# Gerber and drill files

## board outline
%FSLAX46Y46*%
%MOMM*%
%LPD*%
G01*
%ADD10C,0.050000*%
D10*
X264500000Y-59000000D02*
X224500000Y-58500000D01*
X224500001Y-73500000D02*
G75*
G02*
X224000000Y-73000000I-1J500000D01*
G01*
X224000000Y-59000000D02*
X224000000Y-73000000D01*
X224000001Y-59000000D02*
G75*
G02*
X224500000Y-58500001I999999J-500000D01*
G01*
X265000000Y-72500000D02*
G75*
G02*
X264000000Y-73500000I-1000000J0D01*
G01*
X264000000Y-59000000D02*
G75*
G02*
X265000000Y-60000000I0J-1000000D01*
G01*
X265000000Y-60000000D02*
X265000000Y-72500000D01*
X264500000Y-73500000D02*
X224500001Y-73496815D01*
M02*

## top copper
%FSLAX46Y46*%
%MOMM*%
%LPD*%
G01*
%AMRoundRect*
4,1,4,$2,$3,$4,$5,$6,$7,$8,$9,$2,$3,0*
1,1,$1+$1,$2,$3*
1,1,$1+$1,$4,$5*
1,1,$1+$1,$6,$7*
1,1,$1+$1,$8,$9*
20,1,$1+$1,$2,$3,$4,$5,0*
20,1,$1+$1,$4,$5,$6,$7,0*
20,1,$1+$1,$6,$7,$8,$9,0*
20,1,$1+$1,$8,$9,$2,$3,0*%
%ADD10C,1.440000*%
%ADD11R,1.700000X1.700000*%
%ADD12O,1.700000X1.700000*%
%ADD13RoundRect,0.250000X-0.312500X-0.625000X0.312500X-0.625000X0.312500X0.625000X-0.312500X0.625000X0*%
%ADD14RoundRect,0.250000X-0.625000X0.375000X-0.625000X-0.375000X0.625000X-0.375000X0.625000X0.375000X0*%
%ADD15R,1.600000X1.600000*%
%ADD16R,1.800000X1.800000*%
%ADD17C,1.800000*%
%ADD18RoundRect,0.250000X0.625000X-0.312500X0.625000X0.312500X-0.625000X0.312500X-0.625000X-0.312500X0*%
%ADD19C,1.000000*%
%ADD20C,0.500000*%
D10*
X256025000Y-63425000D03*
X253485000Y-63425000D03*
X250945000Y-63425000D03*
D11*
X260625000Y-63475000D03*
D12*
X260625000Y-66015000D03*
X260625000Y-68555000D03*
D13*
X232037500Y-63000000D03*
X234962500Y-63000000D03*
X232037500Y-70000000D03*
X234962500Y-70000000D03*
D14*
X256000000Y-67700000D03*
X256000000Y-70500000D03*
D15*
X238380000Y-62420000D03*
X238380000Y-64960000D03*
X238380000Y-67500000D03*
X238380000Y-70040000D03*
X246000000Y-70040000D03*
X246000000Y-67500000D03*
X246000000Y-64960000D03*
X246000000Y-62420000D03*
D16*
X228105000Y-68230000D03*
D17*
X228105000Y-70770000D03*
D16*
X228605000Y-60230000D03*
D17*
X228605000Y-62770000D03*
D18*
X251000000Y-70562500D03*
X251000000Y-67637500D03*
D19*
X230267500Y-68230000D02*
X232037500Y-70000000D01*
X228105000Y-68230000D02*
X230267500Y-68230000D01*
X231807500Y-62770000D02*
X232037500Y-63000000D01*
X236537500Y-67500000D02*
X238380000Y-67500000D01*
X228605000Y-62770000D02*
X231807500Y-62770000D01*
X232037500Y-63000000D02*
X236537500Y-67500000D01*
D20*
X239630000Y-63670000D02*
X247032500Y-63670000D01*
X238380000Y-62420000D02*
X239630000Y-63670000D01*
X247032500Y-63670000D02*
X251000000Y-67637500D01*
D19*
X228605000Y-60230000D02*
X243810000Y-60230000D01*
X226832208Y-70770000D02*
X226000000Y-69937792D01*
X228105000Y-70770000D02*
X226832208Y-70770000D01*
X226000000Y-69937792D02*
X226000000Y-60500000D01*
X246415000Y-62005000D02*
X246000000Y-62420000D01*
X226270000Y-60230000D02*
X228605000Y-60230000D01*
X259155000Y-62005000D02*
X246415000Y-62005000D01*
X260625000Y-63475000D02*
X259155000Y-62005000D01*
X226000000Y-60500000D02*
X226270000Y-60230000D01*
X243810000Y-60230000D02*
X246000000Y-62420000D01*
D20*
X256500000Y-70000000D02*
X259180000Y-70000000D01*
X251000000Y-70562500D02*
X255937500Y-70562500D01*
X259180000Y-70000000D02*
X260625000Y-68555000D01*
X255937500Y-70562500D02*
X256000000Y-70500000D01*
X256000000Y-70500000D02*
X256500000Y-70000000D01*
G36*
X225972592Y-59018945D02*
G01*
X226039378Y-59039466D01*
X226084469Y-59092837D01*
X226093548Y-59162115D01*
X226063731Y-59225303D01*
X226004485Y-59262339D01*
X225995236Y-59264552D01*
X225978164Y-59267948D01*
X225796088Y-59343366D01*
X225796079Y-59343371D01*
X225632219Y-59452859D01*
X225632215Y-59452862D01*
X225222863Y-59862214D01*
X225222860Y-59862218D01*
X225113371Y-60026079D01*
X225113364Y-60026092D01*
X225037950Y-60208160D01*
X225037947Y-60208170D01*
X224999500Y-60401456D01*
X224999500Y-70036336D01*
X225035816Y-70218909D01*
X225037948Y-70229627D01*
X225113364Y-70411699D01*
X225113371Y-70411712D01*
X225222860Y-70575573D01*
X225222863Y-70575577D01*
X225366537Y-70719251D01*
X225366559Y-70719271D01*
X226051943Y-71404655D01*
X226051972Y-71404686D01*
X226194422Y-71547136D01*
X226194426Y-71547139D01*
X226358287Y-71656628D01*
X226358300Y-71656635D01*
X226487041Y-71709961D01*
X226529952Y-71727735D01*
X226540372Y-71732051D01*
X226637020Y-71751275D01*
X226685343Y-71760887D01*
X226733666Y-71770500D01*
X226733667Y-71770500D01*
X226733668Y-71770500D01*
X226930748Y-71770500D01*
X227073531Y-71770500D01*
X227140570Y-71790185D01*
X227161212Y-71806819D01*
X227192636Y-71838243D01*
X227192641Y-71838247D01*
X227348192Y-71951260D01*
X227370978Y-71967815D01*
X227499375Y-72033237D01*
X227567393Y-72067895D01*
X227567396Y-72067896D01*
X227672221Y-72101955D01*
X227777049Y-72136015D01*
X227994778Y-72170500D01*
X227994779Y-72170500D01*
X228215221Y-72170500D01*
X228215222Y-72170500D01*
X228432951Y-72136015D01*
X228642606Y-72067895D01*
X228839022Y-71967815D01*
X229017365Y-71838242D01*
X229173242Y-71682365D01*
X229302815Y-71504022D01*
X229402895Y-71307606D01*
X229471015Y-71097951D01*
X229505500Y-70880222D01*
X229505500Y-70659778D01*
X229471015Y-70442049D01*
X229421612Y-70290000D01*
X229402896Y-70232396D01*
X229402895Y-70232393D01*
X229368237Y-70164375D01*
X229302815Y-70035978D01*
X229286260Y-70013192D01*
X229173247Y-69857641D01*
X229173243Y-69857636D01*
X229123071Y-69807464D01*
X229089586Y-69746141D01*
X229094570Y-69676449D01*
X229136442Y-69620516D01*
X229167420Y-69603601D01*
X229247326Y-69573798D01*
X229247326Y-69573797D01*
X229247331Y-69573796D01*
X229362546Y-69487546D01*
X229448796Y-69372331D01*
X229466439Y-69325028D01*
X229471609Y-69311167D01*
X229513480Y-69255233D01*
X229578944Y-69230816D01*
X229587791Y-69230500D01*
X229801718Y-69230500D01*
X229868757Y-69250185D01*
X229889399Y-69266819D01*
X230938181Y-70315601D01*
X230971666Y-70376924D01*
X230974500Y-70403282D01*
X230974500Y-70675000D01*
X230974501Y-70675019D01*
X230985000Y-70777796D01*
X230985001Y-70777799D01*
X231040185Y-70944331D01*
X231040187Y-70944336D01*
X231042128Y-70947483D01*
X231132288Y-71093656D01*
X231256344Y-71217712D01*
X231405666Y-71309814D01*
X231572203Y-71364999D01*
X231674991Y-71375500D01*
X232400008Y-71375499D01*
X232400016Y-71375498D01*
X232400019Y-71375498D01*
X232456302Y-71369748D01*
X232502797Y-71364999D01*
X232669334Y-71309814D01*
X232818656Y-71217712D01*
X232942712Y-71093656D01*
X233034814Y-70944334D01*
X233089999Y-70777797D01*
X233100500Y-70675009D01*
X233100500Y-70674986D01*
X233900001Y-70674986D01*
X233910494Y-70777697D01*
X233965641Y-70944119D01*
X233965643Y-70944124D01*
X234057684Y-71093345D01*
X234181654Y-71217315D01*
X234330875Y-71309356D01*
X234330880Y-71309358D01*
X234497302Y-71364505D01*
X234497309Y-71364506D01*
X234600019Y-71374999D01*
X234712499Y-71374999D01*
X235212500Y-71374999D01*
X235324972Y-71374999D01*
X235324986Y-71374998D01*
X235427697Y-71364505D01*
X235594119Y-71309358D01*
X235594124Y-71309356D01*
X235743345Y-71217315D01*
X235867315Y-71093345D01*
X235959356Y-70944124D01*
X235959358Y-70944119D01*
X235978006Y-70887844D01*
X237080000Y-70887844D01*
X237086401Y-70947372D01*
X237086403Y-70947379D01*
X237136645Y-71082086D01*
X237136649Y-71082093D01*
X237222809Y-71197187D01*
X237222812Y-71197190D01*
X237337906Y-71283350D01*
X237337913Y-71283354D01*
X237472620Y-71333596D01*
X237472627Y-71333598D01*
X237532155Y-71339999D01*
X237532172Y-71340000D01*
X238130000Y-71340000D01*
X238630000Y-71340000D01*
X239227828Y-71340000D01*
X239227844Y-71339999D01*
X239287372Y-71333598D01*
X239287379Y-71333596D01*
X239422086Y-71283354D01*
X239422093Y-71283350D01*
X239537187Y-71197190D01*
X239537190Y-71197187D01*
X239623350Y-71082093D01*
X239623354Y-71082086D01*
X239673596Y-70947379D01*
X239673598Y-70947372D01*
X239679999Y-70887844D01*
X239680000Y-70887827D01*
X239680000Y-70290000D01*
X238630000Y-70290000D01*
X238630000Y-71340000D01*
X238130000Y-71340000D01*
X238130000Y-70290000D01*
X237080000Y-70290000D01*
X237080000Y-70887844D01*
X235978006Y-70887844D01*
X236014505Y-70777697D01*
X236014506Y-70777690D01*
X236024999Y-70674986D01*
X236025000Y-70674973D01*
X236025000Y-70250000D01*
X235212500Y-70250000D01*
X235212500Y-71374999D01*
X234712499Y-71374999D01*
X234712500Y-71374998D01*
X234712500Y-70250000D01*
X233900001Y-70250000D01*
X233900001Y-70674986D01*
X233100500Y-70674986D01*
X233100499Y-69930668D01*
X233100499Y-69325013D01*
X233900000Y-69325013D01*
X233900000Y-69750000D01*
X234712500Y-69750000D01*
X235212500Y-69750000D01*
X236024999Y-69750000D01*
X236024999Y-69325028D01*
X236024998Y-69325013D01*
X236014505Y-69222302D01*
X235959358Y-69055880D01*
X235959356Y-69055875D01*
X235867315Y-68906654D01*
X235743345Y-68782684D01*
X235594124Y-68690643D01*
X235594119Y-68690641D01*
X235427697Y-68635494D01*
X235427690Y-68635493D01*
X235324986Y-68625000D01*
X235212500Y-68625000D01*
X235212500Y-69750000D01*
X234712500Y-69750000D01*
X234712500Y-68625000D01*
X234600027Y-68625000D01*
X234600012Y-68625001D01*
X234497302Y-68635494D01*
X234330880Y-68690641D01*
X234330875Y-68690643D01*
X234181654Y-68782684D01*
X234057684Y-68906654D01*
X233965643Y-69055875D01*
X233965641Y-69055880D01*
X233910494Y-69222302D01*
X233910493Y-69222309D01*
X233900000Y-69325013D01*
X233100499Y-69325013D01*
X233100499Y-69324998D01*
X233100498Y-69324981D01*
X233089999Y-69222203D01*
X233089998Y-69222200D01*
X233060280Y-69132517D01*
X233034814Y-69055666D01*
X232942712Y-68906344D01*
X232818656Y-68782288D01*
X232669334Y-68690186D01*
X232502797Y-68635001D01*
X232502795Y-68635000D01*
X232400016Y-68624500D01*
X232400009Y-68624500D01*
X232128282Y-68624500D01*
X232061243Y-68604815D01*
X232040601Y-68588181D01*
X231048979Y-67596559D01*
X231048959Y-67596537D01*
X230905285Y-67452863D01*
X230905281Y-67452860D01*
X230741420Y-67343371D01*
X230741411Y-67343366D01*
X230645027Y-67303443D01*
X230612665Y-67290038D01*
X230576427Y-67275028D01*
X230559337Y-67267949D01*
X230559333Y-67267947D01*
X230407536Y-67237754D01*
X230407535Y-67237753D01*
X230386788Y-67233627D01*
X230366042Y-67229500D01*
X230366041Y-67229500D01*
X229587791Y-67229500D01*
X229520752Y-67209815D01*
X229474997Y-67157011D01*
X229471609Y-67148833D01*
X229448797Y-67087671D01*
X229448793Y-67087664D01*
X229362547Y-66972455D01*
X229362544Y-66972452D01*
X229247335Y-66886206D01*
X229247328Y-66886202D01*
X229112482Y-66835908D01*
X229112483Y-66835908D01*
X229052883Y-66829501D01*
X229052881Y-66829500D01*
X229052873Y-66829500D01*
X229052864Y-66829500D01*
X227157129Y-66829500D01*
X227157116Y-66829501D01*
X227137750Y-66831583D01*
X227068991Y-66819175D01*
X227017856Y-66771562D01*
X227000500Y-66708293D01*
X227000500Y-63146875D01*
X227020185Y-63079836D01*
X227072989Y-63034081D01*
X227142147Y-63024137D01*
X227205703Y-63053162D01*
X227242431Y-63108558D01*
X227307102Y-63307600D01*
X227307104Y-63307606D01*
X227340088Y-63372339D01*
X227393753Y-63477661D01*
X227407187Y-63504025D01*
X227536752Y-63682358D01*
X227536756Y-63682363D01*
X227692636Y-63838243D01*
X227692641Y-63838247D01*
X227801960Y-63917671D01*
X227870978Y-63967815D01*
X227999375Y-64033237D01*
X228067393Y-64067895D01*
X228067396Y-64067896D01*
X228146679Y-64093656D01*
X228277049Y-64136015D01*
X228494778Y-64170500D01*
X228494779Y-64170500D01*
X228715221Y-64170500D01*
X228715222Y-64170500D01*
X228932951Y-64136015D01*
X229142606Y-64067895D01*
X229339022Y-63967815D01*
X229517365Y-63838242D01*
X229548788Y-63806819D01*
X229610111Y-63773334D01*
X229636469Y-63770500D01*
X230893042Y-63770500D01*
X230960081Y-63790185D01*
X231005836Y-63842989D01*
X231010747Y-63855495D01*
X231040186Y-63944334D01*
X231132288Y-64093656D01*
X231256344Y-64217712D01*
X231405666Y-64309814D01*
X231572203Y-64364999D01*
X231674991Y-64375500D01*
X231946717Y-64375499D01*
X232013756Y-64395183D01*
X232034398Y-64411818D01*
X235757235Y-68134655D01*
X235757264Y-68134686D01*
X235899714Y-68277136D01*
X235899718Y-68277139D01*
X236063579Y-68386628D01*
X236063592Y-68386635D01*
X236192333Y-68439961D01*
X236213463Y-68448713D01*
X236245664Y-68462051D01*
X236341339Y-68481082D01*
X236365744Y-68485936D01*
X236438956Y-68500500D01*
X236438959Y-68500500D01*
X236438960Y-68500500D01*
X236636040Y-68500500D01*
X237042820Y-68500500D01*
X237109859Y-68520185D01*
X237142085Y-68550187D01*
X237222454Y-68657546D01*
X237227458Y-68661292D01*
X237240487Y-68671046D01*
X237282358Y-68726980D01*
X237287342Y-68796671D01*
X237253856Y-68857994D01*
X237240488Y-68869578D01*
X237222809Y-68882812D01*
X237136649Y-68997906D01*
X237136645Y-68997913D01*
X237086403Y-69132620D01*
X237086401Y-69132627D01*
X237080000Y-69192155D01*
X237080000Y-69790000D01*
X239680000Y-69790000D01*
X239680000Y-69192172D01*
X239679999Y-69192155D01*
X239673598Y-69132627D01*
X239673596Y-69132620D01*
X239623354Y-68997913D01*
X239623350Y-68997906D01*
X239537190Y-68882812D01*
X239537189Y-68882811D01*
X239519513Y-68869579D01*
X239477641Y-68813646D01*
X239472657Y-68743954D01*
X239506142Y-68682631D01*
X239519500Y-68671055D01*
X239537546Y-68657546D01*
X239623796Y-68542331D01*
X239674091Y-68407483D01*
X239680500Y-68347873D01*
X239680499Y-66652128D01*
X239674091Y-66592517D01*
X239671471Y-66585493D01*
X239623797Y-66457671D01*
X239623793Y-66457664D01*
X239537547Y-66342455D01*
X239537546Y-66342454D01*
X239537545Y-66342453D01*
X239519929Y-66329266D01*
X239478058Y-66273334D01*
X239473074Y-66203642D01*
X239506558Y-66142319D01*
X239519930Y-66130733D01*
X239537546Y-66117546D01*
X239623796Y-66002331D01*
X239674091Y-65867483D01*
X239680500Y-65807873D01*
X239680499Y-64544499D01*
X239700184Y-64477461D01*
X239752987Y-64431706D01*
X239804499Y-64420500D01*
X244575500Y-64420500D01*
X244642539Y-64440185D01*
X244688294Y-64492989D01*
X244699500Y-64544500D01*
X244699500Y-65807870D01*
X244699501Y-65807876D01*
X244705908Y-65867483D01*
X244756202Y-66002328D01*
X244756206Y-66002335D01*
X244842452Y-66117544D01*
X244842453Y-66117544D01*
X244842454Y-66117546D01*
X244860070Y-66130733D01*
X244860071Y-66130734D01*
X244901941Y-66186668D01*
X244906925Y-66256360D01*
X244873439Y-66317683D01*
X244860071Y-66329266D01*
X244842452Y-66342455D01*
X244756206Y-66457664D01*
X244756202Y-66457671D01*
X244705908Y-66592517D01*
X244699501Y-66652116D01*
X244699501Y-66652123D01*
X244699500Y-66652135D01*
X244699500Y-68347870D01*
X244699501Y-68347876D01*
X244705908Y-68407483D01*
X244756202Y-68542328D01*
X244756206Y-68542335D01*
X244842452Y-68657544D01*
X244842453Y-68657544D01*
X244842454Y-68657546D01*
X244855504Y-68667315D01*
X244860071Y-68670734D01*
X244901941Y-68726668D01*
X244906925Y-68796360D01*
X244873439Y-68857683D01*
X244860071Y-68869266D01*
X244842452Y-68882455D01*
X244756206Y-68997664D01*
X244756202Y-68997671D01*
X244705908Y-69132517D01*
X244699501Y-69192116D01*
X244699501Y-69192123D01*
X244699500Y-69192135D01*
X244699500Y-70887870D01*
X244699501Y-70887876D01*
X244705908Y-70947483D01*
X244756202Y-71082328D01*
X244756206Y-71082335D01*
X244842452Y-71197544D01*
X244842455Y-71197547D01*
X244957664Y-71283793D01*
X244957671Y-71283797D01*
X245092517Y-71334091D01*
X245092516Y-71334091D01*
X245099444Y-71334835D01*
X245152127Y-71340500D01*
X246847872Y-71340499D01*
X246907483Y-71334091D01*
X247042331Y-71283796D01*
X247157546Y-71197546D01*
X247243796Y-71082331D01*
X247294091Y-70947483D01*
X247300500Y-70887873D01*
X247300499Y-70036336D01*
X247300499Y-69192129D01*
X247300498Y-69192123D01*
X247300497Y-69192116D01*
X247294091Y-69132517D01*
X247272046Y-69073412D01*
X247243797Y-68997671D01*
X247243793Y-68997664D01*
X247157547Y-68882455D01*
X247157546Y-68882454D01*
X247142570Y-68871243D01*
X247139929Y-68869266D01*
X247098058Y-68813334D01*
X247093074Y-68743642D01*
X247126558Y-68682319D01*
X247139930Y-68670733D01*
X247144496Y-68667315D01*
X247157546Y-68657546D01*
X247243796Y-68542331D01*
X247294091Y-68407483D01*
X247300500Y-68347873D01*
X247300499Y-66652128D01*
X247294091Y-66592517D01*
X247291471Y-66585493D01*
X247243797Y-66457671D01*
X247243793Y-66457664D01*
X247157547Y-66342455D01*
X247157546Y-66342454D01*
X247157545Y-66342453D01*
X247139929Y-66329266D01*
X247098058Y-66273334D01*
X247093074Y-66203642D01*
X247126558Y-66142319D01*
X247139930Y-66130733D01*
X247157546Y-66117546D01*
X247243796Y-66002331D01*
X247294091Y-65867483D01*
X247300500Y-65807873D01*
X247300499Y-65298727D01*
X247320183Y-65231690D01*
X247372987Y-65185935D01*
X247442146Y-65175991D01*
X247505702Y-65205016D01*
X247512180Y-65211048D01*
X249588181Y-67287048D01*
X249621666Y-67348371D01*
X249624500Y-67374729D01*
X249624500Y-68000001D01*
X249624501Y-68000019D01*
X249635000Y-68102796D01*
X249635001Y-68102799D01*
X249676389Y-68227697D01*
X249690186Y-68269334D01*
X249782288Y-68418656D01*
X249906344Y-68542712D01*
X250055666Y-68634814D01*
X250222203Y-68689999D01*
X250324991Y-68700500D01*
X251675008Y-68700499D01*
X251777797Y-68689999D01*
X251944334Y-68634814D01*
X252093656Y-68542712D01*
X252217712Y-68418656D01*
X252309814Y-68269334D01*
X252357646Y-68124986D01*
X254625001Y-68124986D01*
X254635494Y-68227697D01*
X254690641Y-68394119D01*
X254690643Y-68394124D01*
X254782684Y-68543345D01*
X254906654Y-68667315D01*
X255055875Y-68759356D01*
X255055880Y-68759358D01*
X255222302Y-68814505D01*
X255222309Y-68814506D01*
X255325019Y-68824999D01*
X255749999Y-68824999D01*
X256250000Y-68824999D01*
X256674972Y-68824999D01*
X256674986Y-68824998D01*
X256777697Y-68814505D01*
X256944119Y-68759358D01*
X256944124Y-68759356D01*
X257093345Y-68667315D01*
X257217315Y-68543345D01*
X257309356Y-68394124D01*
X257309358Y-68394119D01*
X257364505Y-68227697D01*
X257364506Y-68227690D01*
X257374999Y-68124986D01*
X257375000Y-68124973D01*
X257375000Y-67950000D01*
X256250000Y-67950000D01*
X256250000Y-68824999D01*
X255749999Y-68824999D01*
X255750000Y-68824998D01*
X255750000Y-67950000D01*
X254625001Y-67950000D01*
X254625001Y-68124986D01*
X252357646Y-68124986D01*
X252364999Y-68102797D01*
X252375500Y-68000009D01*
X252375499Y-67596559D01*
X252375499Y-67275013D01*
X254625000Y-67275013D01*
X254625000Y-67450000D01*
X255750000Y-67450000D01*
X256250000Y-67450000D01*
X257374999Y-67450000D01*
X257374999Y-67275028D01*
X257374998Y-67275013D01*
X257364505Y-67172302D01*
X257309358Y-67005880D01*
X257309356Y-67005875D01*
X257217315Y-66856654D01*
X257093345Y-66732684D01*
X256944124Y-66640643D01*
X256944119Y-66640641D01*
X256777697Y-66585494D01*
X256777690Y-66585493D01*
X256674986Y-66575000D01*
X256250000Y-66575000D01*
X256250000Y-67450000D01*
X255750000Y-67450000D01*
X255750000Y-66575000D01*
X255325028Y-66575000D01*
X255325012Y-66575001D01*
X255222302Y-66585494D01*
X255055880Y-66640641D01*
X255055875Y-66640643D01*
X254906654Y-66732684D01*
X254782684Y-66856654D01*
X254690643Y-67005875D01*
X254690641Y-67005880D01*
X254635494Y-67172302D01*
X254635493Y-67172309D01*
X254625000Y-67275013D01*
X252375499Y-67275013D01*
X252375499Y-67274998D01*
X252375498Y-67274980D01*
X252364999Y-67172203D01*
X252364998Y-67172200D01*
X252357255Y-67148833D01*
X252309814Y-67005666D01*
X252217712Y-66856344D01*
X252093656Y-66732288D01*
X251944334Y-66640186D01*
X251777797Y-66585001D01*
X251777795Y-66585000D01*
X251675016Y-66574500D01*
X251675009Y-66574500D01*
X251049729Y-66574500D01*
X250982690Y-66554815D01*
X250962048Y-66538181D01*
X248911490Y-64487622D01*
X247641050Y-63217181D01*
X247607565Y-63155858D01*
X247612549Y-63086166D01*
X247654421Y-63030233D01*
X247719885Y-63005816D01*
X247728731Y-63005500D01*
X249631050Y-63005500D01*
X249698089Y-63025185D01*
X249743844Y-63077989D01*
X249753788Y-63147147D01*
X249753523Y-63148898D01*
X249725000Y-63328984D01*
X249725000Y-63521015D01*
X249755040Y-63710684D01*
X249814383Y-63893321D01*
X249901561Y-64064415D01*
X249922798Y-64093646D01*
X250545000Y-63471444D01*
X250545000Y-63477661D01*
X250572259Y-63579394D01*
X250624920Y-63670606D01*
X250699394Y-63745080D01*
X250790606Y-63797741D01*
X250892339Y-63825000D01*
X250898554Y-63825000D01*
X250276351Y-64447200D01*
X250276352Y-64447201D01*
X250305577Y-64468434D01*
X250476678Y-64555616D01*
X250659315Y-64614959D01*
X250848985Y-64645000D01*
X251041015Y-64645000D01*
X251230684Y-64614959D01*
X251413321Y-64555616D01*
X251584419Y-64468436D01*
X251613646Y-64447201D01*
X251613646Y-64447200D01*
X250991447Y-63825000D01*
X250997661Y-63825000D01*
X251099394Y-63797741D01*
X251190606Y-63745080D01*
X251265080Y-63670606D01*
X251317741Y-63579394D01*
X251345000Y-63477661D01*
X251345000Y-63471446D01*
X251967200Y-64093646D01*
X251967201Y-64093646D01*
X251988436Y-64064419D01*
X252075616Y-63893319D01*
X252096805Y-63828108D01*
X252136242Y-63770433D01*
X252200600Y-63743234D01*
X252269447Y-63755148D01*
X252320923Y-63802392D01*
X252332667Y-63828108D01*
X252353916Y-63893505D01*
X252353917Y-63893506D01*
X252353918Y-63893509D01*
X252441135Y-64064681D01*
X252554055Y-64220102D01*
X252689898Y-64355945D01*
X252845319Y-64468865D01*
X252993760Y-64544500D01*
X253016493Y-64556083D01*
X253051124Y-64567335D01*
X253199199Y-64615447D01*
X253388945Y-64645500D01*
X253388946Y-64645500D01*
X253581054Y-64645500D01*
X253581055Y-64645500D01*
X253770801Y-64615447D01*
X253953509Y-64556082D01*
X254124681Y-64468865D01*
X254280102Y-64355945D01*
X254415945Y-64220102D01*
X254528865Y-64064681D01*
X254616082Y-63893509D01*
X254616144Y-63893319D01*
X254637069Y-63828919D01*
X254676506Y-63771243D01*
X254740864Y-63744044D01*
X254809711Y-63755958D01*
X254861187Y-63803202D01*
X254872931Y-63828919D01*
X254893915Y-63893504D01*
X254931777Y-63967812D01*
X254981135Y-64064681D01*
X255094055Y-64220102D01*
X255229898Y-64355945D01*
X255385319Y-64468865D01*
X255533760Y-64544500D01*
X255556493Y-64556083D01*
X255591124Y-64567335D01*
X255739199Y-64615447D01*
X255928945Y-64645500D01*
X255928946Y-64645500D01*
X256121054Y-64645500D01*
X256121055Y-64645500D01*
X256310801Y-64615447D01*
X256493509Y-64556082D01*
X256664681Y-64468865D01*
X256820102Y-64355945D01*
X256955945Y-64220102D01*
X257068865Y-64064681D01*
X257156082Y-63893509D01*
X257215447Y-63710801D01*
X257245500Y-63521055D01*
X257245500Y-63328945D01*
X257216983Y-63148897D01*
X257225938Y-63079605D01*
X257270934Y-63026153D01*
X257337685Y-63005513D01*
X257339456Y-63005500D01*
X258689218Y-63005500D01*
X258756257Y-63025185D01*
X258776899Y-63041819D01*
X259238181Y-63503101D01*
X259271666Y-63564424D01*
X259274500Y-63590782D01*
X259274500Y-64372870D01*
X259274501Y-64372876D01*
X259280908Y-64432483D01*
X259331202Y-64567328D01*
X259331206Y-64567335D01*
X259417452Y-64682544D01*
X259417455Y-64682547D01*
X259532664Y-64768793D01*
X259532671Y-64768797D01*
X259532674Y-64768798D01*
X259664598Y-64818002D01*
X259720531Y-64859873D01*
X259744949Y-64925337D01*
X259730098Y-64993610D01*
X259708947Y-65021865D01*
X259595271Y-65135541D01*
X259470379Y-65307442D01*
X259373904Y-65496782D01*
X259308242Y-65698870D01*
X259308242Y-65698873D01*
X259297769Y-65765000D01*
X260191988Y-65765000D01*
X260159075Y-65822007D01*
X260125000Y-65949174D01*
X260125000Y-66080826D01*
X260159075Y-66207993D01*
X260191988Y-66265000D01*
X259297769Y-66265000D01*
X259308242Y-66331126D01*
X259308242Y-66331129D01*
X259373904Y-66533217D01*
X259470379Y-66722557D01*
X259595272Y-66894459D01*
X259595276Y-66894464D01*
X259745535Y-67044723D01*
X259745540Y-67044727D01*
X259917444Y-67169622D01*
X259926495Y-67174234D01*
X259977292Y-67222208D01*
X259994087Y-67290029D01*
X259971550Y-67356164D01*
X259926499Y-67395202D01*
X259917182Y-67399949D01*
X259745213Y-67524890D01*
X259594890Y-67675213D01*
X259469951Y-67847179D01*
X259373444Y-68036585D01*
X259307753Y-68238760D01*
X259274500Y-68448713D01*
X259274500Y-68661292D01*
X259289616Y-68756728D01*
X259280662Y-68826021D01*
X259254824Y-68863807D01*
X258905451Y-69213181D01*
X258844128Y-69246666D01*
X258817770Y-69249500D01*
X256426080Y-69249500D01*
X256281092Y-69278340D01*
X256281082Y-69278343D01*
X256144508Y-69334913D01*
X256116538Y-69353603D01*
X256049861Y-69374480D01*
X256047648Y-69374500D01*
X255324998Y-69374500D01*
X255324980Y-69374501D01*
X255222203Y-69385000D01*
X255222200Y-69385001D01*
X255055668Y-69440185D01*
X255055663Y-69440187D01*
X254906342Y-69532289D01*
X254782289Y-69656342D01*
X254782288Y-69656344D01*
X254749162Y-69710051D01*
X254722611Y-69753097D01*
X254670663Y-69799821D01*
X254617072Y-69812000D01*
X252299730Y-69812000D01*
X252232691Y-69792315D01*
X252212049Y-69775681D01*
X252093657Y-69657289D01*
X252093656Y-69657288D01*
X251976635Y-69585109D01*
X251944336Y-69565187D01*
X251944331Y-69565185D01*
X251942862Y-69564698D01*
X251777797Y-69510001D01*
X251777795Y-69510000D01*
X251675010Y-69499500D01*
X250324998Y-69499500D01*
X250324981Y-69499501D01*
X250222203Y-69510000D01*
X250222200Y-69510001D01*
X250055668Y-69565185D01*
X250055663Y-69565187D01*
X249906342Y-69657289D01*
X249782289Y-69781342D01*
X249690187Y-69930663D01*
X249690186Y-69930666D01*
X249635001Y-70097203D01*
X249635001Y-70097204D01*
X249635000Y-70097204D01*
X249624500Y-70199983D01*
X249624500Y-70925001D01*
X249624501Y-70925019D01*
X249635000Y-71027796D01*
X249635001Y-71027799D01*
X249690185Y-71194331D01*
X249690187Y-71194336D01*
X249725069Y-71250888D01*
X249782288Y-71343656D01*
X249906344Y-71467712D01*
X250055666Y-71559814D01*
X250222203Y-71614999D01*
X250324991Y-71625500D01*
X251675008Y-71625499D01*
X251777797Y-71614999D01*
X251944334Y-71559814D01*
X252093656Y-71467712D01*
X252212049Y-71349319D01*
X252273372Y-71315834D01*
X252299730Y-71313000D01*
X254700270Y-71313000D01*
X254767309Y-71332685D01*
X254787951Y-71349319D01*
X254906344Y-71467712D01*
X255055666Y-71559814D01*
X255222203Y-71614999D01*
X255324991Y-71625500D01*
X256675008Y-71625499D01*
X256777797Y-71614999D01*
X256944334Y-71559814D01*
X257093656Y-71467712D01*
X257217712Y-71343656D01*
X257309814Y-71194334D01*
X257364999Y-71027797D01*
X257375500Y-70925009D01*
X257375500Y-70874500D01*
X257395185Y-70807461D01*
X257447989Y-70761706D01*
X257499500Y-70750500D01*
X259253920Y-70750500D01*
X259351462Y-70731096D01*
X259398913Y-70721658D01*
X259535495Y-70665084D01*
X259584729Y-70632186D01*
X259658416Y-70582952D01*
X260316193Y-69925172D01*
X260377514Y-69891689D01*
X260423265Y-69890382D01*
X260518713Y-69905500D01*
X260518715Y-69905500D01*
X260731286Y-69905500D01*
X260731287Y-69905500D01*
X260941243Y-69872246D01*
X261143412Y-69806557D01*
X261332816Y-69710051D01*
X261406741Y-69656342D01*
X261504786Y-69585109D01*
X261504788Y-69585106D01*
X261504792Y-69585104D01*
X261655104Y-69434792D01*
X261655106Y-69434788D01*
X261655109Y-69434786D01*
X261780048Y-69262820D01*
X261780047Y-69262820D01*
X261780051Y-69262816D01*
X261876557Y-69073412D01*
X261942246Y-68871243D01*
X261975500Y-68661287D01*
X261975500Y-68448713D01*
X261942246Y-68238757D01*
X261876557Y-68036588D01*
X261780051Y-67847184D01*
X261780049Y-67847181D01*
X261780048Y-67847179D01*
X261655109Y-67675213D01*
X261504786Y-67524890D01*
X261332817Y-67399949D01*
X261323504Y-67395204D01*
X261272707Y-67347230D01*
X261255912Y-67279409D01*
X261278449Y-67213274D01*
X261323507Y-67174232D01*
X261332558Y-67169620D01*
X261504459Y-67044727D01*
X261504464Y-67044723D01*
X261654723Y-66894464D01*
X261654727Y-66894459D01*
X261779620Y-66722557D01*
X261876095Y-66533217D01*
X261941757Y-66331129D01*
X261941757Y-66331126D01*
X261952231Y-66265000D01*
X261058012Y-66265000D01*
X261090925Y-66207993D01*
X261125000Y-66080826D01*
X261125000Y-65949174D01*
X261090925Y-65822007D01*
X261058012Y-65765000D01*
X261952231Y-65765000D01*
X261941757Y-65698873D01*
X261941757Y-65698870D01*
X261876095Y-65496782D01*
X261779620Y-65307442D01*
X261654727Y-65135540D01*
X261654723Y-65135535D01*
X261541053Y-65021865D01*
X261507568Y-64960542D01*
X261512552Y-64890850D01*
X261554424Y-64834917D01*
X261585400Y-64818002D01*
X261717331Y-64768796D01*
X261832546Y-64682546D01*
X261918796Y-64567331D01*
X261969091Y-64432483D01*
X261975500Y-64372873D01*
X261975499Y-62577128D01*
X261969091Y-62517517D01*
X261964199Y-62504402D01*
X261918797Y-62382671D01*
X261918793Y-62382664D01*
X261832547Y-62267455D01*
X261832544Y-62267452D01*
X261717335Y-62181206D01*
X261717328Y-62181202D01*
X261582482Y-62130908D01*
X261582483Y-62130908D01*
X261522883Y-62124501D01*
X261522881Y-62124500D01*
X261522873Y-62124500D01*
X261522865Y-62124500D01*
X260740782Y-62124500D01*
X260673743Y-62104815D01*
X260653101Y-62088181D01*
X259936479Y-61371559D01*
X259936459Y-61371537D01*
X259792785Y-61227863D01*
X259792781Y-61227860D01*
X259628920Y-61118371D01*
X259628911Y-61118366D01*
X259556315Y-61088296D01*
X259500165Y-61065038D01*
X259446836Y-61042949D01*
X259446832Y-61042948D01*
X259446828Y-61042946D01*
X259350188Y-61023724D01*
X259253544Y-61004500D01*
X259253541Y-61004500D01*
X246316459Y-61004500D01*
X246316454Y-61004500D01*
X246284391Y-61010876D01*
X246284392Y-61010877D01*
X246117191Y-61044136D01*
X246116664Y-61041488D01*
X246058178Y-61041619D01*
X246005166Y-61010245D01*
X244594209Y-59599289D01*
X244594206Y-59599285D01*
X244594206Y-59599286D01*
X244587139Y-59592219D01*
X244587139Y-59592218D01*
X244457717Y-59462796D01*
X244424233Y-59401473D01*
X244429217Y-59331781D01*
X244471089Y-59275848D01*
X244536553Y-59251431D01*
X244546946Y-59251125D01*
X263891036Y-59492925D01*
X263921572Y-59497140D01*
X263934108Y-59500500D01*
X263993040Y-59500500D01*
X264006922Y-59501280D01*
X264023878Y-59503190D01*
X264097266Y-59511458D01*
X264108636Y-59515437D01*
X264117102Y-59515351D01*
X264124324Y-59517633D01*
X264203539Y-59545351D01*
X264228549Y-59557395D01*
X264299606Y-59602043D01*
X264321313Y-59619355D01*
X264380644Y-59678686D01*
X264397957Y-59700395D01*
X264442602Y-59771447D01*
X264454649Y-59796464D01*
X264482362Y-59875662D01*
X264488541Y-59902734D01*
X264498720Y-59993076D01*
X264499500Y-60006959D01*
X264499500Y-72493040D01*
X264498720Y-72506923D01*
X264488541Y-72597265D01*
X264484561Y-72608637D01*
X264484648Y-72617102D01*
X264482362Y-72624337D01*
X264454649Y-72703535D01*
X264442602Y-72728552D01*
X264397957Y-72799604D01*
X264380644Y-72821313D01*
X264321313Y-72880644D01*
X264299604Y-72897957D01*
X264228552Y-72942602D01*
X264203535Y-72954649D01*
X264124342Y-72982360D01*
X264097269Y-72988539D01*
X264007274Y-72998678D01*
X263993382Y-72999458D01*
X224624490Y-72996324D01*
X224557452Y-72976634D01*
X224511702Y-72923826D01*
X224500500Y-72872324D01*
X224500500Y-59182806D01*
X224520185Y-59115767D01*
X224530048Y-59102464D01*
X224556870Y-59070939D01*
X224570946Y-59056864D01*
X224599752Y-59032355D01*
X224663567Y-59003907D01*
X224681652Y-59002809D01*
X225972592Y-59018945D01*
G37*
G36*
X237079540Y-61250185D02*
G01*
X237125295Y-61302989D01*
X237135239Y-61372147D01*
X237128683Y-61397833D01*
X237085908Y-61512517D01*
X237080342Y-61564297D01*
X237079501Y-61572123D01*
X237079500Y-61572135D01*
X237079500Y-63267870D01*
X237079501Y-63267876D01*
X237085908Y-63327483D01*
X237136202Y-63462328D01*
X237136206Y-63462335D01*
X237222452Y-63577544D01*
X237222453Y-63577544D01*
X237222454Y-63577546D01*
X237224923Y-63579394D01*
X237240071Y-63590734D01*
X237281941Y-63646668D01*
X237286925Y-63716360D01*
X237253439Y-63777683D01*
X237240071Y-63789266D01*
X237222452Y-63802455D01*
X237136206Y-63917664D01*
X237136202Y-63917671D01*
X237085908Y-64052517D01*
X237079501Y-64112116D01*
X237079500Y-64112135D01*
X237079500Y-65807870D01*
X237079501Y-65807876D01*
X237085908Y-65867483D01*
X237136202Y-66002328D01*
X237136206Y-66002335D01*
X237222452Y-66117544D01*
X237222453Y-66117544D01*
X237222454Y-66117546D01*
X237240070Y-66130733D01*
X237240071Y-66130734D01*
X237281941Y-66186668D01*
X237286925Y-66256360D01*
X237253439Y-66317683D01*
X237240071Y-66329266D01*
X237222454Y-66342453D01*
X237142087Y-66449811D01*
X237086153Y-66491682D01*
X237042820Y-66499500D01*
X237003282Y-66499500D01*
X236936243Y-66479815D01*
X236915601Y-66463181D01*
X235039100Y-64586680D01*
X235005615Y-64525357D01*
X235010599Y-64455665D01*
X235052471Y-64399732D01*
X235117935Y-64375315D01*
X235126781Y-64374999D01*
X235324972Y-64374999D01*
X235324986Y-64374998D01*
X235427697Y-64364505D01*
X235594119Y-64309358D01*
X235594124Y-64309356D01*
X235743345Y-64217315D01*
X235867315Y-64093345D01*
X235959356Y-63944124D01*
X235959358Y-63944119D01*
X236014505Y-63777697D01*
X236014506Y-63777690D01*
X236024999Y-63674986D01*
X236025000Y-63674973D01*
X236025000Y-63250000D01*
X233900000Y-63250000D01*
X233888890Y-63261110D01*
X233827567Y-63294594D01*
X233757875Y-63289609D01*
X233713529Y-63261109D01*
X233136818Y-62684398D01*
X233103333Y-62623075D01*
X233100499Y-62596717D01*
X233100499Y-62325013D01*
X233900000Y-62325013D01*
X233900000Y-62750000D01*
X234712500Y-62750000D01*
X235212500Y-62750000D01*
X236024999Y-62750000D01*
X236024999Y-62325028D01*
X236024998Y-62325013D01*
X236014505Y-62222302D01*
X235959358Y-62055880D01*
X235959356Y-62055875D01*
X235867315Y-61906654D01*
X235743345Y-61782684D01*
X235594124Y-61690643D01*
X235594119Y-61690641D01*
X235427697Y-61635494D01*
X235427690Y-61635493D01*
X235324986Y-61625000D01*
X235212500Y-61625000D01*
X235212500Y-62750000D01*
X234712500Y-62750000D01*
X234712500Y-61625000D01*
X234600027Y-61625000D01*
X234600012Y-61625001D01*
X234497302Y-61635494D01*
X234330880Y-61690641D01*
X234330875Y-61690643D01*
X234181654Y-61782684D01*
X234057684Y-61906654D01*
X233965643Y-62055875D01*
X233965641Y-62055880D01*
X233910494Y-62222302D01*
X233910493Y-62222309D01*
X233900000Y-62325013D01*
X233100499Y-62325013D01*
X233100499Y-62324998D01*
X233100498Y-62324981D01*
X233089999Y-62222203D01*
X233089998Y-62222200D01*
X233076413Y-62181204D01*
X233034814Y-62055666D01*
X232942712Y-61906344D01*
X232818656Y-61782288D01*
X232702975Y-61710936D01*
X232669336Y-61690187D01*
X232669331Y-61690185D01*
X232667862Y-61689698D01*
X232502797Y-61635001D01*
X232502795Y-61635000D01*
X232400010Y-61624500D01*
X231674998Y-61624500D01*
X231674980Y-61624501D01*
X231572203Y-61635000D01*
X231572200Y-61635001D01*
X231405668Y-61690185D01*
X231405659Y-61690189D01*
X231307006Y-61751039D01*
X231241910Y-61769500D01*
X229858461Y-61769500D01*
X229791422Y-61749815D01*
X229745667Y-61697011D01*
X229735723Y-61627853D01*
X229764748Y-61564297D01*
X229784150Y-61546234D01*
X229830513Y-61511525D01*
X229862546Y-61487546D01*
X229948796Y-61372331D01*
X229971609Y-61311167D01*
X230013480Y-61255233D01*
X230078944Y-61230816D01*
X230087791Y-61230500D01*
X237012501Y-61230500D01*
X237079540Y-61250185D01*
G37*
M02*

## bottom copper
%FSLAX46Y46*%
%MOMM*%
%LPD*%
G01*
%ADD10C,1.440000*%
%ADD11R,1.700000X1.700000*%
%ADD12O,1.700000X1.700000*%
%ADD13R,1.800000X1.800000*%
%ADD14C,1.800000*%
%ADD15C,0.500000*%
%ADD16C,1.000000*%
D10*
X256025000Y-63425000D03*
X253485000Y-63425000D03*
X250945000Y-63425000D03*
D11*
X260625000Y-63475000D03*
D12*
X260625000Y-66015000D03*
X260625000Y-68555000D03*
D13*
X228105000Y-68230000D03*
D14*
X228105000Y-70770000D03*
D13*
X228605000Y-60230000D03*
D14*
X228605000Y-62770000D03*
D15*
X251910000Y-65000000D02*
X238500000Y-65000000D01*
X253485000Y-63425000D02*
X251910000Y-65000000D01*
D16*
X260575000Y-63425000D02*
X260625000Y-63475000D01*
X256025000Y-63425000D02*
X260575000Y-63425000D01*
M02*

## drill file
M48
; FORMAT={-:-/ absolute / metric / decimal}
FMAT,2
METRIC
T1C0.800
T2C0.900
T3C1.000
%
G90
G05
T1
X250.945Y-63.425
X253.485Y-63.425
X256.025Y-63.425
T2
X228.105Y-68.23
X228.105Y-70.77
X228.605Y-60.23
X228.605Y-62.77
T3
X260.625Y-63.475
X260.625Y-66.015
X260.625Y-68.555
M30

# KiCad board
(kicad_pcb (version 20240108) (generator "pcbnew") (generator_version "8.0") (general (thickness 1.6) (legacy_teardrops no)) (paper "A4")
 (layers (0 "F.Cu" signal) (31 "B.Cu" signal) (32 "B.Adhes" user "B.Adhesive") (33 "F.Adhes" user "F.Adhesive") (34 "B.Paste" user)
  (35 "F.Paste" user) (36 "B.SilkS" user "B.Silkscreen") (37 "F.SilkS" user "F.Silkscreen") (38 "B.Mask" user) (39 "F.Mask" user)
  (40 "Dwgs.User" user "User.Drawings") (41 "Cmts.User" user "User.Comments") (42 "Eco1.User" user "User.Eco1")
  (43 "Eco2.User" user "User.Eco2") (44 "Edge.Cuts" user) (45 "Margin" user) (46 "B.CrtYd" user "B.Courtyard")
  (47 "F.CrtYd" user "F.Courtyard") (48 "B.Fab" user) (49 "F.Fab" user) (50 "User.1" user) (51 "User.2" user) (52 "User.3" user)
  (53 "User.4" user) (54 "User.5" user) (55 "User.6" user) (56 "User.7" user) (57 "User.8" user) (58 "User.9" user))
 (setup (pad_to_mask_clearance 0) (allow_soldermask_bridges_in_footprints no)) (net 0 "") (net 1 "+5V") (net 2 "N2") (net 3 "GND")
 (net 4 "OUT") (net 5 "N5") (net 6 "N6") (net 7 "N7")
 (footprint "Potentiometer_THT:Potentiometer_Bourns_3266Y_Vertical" (layer "F.Cu") (at 256.025 63.425)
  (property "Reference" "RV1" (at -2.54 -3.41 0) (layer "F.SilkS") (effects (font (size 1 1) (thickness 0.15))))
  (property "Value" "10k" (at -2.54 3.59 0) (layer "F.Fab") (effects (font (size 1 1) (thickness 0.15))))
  (pad "1" thru_hole circle (at 0 0) (size 1.44 1.44) (drill 0.8) (layers "*.Cu" "*.Mask") (remove_unused_layers no) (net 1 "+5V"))
  (pad "2" thru_hole circle (at -2.54 0) (size 1.44 1.44) (drill 0.8) (layers "*.Cu" "*.Mask") (remove_unused_layers no) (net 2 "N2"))
  (pad "3" thru_hole circle (at -5.08 0) (size 1.44 1.44) (drill 0.8) (layers "*.Cu" "*.Mask") (remove_unused_layers no) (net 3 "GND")))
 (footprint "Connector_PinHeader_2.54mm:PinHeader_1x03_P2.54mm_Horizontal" (layer "F.Cu") (at 260.625 63.475)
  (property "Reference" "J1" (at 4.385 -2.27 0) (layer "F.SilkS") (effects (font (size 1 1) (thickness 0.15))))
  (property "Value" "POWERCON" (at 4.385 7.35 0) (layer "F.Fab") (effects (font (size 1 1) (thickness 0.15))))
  (pad "1" thru_hole rect (at 0 0) (size 1.7 1.7) (drill 1) (layers "*.Cu" "*.Mask") (remove_unused_layers no) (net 1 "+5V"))
  (pad "2" thru_hole oval (at 0 2.54) (size 1.7 1.7) (drill 1) (layers "*.Cu" "*.Mask") (remove_unused_layers no) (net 3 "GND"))
  (pad "3" thru_hole oval (at 0 5.08) (size 1.7 1.7) (drill 1) (layers "*.Cu" "*.Mask") (remove_unused_layers no) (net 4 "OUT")))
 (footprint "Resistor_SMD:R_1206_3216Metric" (layer "F.Cu") (at 233.5 63)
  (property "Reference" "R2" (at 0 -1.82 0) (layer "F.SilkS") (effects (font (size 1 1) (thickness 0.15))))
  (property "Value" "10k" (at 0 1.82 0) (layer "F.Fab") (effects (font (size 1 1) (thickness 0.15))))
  (pad "1" smd roundrect (at -1.4625 0) (size 1.125 1.75) (layers "F.Cu" "F.Paste" "F.Mask") (roundrect_rratio 0.222222) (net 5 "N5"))
  (pad "2" smd roundrect (at 1.4625 0) (size 1.125 1.75) (layers "F.Cu" "F.Paste" "F.Mask") (roundrect_rratio 0.222222) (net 3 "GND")))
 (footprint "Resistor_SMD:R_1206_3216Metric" (layer "F.Cu") (at 233.5 70)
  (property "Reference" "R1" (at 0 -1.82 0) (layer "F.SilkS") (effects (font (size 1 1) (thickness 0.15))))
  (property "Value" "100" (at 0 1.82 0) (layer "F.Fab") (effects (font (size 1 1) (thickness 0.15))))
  (pad "1" smd roundrect (at -1.4625 0) (size 1.125 1.75) (layers "F.Cu" "F.Paste" "F.Mask") (roundrect_rratio 0.222222) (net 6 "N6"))
  (pad "2" smd roundrect (at 1.4625 0) (size 1.125 1.75) (layers "F.Cu" "F.Paste" "F.Mask") (roundrect_rratio 0.222222) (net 3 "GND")))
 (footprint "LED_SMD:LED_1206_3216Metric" (layer "F.Cu") (at 256 69.1 -90)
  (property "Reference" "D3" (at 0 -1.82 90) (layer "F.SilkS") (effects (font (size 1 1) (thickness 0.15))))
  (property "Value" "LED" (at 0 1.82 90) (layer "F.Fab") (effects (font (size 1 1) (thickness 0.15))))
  (pad "1" smd roundrect (at -1.4 0 270) (size 1.25 1.75) (layers "F.Cu" "F.Paste" "F.Mask") (roundrect_rratio 0.2) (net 3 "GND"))
  (pad "2" smd roundrect (at 1.4 0 270) (size 1.25 1.75) (layers "F.Cu" "F.Paste" "F.Mask") (roundrect_rratio 0.2) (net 4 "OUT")))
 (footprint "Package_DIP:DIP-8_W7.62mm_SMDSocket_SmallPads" (layer "F.Cu") (at 242.19 66.23)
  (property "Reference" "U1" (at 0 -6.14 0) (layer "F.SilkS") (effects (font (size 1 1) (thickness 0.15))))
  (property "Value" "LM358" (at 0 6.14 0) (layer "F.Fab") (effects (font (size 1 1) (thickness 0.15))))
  (pad "1" smd rect (at -3.81 -3.81) (size 1.6 1.6) (layers "F.Cu" "F.Paste" "F.Mask") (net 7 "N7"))
  (pad "2" smd rect (at -3.81 -1.27) (size 1.6 1.6) (layers "F.Cu" "F.Paste" "F.Mask") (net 2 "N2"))
  (pad "3" smd rect (at -3.81 1.27) (size 1.6 1.6) (layers "F.Cu" "F.Paste" "F.Mask") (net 5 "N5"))
  (pad "4" smd rect (at -3.81 3.81) (size 1.6 1.6) (layers "F.Cu" "F.Paste" "F.Mask") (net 3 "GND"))
  (pad "5" smd rect (at 3.81 3.81) (size 1.6 1.6) (layers "F.Cu" "F.Paste" "F.Mask"))
  (pad "6" smd rect (at 3.81 1.27) (size 1.6 1.6) (layers "F.Cu" "F.Paste" "F.Mask"))
  (pad "7" smd rect (at 3.81 -1.27) (size 1.6 1.6) (layers "F.Cu" "F.Paste" "F.Mask"))
  (pad "8" smd rect (at 3.81 -3.81) (size 1.6 1.6) (layers "F.Cu" "F.Paste" "F.Mask") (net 1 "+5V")))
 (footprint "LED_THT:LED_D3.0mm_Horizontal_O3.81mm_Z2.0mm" (layer "F.Cu") (at 228.105 68.23 -90)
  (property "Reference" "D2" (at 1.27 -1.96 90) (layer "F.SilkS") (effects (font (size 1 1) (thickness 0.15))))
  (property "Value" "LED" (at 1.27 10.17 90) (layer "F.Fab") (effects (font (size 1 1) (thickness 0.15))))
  (pad "1" thru_hole rect (at 0 0 270) (size 1.8 1.8) (drill 0.9) (layers "*.Cu" "*.Mask") (remove_unused_layers no) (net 6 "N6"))
  (pad "2" thru_hole circle (at 2.54 0 270) (size 1.8 1.8) (drill 0.9) (layers "*.Cu" "*.Mask") (remove_unused_layers no) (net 1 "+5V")))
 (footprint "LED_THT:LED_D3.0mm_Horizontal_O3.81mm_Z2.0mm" (layer "F.Cu") (at 228.605 60.23 -90)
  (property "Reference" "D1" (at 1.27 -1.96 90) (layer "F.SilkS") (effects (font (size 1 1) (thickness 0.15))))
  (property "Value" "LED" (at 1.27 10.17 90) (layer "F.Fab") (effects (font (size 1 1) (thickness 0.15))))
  (pad "1" thru_hole rect (at 0 0 270) (size 1.8 1.8) (drill 0.9) (layers "*.Cu" "*.Mask") (remove_unused_layers no) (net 1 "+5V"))
  (pad "2" thru_hole circle (at 2.54 0 270) (size 1.8 1.8) (drill 0.9) (layers "*.Cu" "*.Mask") (remove_unused_layers no) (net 5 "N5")))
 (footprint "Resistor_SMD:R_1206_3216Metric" (layer "F.Cu") (at 251 69.1 90)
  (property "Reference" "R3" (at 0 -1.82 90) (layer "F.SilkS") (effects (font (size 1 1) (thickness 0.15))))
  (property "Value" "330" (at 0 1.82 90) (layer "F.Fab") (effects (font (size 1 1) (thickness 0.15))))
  (pad "1" smd roundrect (at -1.4625 0 90) (size 1.125 1.75) (layers "F.Cu" "F.Paste" "F.Mask") (roundrect_rratio 0.222222) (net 4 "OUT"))
  (pad "2" smd roundrect (at 1.4625 0 90) (size 1.125 1.75) (layers "F.Cu" "F.Paste" "F.Mask") (roundrect_rratio 0.222222) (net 7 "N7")))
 (gr_line (start 264.5 59) (end 224.5 58.5) (stroke (width 0.05) (type default)) (layer "Edge.Cuts"))
 (gr_arc (start 224.500001 73.5) (mid 224.146447 73.353554) (end 224 73) (stroke (width 0.05) (type default)) (layer "Edge.Cuts"))
 (gr_line (start 224 59) (end 224 73) (stroke (width 0.05) (type default)) (layer "Edge.Cuts"))
 (gr_arc (start 224.000001 59) (mid 224.209431 58.709431) (end 224.5 58.500001) (stroke (width 0.05) (type default)) (layer "Edge.Cuts"))
 (gr_arc (start 265 72.5) (mid 264.707107 73.207107) (end 264 73.5) (stroke (width 0.05) (type default)) (layer "Edge.Cuts"))
 (gr_arc (start 264 59) (mid 264.707107 59.292893) (end 265 60) (stroke (width 0.05) (type default)) (layer "Edge.Cuts"))
 (gr_line (start 265 60) (end 265 72.5) (stroke (width 0.05) (type default)) (layer "Edge.Cuts"))
 (gr_line (start 264.5 73.5) (end 224.500001 73.496815) (stroke (width 0.05) (type default)) (layer "Edge.Cuts"))
 (segment (start 230.2675 68.23) (end 232.0375 70) (width 1) (layer "F.Cu") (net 6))
 (segment (start 228.105 68.23) (end 230.2675 68.23) (width 1) (layer "F.Cu") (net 6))
 (segment (start 231.8075 62.77) (end 232.0375 63) (width 1) (layer "F.Cu") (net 5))
 (segment (start 236.5375 67.5) (end 238.38 67.5) (width 1) (layer "F.Cu") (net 5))
 (segment (start 228.605 62.77) (end 231.8075 62.77) (width 1) (layer "F.Cu") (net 5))
 (segment (start 232.0375 63) (end 236.5375 67.5) (width 1) (layer "F.Cu") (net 5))
 (segment (start 239.63 63.67) (end 247.0325 63.67) (width 0.5) (layer "F.Cu") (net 7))
 (segment (start 238.38 62.42) (end 239.63 63.67) (width 0.5) (layer "F.Cu") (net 7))
 (segment (start 247.0325 63.67) (end 251 67.6375) (width 0.5) (layer "F.Cu") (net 7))
 (segment (start 251.91 65) (end 238.5 65) (width 0.5) (layer "B.Cu") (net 2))
 (segment (start 253.485 63.425) (end 251.91 65) (width 0.5) (layer "B.Cu") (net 2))
 (segment (start 228.605 60.23) (end 243.81 60.23) (width 1) (layer "F.Cu") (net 1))
 (segment (start 226.832208 70.77) (end 226 69.937792) (width 1) (layer "F.Cu") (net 1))
 (segment (start 228.105 70.77) (end 226.832208 70.77) (width 1) (layer "F.Cu") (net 1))
 (segment (start 226 69.937792) (end 226 60.5) (width 1) (layer "F.Cu") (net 1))
 (segment (start 246.415 62.005) (end 246 62.42) (width 1) (layer "F.Cu") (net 1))
 (segment (start 226.27 60.23) (end 228.605 60.23) (width 1) (layer "F.Cu") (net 1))
 (segment (start 259.155 62.005) (end 246.415 62.005) (width 1) (layer "F.Cu") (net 1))
 (segment (start 260.625 63.475) (end 259.155 62.005) (width 1) (layer "F.Cu") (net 1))
 (segment (start 226 60.5) (end 226.27 60.23) (width 1) (layer "F.Cu") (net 1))
 (segment (start 243.81 60.23) (end 246 62.42) (width 1) (layer "F.Cu") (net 1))
 (segment (start 260.575 63.425) (end 260.625 63.475) (width 1) (layer "B.Cu") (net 1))
 (segment (start 256.025 63.425) (end 260.575 63.425) (width 1) (layer "B.Cu") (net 1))
 (segment (start 256.5 70) (end 259.18 70) (width 0.5) (layer "F.Cu") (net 4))
 (segment (start 251 70.5625) (end 255.9375 70.5625) (width 0.5) (layer "F.Cu") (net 4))
 (segment (start 259.18 70) (end 260.625 68.555) (width 0.5) (layer "F.Cu") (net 4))
 (segment (start 255.9375 70.5625) (end 256 70.5) (width 0.5) (layer "F.Cu") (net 4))
 (segment (start 256 70.5) (end 256.5 70) (width 0.5) (layer "F.Cu") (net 4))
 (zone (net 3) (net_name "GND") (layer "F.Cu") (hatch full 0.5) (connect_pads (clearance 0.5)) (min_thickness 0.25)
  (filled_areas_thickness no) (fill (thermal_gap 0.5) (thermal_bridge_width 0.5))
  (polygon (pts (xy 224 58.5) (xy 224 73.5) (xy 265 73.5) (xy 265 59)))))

